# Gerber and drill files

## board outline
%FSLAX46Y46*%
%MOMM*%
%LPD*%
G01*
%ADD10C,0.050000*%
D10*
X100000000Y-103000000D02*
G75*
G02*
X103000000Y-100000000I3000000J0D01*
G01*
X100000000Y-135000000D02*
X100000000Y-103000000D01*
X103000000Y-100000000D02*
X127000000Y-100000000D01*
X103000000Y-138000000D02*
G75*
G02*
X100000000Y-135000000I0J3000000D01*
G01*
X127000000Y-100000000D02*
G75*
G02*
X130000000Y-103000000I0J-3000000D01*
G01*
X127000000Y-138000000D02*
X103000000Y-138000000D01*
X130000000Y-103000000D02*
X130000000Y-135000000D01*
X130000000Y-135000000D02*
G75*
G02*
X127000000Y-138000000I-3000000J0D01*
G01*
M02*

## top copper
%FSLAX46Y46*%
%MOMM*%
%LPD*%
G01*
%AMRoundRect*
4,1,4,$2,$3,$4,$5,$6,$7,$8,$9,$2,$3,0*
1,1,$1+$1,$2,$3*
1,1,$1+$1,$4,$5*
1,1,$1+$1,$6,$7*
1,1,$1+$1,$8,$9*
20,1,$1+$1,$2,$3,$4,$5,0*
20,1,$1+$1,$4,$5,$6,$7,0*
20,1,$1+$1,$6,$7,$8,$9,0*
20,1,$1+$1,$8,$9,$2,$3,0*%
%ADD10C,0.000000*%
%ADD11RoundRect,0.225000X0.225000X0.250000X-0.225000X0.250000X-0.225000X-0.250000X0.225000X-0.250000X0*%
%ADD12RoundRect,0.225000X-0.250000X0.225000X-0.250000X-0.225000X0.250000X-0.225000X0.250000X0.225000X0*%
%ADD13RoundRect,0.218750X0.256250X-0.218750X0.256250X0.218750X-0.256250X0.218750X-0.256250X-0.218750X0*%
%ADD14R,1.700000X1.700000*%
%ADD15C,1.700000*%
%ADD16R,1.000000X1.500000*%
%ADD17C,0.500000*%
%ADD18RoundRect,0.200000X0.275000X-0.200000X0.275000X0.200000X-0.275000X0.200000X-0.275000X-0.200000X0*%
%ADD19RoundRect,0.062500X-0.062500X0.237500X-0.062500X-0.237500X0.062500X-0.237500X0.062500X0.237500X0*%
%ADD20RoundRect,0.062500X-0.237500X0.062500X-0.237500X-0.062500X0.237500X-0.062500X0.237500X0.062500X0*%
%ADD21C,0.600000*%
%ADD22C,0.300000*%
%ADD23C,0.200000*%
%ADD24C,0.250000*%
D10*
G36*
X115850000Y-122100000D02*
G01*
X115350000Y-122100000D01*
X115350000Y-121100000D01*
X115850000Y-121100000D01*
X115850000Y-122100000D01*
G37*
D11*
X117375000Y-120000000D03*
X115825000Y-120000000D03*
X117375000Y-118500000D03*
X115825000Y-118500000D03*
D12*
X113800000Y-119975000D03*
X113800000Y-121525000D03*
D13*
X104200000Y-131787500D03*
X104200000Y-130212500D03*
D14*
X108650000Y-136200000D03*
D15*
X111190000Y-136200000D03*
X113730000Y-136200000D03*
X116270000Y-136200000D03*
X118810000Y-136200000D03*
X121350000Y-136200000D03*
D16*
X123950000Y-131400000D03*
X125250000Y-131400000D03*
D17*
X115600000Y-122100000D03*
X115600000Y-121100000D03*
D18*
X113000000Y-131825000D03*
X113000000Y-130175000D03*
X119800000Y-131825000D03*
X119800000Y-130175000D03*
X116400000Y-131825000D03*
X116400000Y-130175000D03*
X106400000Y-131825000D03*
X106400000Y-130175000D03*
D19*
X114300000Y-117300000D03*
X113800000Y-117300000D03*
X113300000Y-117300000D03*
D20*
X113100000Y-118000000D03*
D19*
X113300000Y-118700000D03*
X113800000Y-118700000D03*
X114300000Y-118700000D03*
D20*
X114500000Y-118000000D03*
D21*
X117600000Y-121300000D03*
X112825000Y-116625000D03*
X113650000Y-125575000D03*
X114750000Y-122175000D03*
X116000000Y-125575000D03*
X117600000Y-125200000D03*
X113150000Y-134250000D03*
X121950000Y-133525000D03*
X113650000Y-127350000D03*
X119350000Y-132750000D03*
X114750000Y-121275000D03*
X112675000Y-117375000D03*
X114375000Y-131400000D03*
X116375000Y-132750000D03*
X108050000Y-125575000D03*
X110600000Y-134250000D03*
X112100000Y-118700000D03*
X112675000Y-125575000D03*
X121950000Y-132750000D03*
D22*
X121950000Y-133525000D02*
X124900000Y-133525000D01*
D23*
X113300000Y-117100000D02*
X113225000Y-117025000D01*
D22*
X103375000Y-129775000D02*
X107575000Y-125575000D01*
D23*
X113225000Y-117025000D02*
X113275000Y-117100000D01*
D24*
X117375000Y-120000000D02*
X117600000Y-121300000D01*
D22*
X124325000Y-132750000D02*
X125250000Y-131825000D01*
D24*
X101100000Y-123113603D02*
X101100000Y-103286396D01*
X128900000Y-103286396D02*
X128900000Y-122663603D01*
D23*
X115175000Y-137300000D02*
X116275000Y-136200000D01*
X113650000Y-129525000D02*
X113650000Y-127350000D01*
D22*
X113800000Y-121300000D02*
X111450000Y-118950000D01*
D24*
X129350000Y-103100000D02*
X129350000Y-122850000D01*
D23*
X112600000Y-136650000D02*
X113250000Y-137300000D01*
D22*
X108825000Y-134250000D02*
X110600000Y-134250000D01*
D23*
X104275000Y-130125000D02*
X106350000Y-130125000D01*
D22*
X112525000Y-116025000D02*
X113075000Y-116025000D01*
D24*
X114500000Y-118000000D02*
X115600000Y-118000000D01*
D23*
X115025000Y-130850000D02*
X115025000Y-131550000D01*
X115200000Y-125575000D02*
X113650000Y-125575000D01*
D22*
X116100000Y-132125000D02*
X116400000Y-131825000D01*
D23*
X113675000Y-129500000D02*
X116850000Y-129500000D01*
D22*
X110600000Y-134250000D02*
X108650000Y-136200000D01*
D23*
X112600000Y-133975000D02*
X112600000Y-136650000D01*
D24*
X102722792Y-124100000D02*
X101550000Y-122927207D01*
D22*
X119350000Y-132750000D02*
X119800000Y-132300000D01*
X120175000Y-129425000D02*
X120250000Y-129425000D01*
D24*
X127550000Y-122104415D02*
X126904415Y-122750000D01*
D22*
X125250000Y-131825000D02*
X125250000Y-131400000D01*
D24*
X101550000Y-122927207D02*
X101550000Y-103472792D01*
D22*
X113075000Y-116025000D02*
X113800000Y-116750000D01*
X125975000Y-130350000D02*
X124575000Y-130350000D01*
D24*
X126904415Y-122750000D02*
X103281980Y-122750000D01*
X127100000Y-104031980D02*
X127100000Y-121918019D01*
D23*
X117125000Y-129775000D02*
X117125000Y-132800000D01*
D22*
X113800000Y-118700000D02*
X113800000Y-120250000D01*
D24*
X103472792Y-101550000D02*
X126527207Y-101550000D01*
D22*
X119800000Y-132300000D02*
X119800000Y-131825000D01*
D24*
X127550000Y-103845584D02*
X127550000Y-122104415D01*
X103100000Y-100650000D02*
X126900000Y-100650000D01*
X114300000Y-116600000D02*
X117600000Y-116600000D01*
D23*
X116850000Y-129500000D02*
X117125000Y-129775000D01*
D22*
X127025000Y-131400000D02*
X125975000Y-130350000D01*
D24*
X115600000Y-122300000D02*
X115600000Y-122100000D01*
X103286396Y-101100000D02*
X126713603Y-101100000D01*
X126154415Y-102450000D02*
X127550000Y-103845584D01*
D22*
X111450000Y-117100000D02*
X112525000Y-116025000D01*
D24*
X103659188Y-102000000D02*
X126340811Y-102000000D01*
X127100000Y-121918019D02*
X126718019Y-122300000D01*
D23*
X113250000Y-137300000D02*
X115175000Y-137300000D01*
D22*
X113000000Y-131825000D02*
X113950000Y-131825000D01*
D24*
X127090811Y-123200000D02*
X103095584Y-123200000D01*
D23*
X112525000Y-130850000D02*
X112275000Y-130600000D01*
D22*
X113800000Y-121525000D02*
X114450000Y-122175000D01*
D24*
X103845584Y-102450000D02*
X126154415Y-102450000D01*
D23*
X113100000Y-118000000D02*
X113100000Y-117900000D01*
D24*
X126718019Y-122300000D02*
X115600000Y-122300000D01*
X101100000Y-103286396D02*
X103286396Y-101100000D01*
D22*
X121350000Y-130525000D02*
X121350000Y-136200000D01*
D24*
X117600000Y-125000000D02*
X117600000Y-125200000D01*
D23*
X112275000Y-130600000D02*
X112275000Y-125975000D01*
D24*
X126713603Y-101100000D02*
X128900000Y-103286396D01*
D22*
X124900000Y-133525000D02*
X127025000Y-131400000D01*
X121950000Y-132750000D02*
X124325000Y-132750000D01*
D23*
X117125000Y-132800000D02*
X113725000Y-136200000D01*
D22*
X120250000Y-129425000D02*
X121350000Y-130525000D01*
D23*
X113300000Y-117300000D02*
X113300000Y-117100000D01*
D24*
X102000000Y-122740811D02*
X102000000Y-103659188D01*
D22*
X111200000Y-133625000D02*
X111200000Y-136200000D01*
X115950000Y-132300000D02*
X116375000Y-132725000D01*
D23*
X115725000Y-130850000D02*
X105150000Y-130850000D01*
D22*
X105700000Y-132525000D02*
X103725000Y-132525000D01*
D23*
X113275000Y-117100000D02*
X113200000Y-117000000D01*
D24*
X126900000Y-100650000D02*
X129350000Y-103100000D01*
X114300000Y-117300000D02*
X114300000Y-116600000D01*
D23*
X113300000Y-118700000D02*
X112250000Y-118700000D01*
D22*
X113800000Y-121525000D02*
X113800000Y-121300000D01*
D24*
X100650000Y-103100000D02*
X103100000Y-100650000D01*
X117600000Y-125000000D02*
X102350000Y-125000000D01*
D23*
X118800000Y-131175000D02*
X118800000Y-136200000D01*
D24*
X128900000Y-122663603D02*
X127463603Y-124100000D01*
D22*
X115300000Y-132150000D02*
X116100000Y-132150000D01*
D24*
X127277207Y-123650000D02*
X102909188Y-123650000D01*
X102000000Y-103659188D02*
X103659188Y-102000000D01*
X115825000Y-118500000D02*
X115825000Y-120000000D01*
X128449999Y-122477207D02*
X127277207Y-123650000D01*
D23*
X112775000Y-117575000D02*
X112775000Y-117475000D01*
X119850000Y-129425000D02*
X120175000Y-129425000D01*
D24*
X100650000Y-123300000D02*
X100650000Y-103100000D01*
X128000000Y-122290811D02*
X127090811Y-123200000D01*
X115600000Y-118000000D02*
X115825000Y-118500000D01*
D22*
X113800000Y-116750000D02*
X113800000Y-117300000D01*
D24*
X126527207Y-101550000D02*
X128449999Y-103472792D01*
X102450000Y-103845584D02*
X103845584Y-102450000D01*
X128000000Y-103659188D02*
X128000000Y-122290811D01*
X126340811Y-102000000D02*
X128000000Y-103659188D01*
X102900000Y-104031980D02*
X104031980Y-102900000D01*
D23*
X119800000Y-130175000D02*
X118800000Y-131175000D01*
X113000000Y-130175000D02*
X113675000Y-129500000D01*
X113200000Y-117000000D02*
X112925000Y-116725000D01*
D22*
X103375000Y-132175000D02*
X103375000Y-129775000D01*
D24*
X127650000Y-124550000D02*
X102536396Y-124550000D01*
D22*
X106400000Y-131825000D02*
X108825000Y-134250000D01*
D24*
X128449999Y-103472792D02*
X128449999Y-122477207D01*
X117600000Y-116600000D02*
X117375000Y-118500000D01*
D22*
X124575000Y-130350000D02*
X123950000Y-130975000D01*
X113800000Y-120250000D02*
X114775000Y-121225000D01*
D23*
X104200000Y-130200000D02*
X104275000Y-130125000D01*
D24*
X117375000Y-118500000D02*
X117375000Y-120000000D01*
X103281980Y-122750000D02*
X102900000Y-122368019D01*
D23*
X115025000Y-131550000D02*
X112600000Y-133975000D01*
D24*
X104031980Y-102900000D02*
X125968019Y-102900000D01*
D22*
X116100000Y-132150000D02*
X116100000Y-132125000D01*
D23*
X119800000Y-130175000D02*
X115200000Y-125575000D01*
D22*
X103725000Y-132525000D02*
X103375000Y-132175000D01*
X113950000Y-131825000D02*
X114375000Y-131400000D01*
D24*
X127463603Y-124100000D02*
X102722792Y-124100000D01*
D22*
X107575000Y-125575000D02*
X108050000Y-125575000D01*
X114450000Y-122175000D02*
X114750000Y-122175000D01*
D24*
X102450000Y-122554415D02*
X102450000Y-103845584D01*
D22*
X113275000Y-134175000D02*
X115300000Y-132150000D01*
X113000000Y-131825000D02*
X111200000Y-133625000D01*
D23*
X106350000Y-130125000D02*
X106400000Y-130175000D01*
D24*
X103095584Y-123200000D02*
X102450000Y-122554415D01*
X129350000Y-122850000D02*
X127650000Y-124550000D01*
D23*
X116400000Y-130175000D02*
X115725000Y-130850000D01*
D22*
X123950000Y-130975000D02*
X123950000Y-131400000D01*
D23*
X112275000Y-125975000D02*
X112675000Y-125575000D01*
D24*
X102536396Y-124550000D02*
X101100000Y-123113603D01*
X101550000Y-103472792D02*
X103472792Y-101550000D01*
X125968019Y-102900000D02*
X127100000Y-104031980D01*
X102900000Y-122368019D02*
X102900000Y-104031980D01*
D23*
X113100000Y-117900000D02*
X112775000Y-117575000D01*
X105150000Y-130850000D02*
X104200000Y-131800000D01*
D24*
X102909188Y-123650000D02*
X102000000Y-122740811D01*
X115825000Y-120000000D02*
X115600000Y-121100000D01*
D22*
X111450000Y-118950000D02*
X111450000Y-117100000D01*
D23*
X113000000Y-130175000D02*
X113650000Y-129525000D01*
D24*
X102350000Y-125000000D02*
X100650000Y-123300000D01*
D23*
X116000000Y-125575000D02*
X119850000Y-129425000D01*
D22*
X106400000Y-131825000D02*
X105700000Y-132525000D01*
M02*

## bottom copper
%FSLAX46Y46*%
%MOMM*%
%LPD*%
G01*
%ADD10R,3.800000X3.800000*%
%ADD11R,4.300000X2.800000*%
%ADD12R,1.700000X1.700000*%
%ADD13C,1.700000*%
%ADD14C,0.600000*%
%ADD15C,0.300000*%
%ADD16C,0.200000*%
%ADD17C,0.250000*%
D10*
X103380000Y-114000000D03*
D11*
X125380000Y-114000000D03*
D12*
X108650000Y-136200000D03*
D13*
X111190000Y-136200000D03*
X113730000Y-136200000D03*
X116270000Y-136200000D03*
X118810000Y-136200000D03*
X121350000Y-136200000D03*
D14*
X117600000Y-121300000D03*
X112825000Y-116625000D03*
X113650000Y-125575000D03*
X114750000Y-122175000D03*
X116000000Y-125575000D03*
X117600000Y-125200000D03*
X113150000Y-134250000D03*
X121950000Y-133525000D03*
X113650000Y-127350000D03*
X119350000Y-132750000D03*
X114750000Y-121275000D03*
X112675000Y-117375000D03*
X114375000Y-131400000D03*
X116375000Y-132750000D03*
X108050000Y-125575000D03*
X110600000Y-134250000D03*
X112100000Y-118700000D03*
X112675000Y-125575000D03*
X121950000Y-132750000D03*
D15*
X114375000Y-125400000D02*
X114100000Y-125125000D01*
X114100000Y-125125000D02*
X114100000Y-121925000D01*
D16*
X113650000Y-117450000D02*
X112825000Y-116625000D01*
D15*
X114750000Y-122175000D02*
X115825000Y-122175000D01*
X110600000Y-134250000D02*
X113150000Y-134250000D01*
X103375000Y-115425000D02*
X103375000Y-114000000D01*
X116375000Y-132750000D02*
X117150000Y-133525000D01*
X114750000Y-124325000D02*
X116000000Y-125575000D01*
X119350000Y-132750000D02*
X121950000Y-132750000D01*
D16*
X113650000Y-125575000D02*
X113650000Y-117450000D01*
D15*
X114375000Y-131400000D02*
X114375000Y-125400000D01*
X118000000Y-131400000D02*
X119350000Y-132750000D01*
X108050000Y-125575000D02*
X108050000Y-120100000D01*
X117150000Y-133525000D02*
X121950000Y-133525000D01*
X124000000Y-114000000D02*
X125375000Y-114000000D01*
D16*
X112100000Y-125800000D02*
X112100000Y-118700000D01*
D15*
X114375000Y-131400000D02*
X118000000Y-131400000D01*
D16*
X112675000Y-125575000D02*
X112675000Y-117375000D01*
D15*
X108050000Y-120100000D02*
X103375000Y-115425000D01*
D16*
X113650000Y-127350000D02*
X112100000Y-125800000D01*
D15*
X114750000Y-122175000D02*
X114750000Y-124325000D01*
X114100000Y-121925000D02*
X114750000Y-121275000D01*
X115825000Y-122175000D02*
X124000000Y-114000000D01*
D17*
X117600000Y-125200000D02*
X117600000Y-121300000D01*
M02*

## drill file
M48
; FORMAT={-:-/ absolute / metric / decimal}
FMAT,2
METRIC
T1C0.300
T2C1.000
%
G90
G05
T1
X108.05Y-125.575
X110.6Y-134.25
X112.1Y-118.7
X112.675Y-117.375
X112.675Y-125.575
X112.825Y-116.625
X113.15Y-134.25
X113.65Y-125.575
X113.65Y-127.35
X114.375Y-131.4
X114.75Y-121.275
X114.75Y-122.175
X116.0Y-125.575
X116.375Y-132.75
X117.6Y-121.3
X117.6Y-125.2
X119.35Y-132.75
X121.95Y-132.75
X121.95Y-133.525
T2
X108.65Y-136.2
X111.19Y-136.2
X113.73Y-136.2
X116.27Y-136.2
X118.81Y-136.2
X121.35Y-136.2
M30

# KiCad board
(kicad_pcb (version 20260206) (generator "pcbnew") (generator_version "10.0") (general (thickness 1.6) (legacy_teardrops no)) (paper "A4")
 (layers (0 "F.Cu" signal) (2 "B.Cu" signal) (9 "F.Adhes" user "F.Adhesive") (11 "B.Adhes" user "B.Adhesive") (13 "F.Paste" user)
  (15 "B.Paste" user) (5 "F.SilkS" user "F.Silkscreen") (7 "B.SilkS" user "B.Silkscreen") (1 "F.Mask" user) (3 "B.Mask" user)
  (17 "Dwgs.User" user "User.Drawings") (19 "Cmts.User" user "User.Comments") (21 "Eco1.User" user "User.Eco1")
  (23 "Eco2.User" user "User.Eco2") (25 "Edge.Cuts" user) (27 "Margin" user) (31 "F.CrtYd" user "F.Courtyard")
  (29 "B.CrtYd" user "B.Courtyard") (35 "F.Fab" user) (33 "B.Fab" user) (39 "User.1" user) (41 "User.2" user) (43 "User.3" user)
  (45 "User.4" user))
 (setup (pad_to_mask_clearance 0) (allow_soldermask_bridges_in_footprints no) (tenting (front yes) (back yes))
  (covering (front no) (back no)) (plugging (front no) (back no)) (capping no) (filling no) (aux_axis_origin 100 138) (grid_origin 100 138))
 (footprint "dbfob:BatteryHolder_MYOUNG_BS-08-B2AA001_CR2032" (layer "B.Cu") (at 114.4 114 180)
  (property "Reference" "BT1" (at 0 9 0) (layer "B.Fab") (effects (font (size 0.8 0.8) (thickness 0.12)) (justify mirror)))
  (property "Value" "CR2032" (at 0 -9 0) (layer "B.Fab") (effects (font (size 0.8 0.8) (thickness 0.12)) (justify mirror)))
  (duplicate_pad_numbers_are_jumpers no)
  (pad "1" smd rect (at 11.02 0 180) (size 3.8 3.8) (layers "B.Cu" "B.Mask" "B.Paste") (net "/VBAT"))
  (pad "2" smd rect (at -10.98 0 180) (size 4.3 2.8) (layers "B.Cu" "B.Mask" "B.Paste") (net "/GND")))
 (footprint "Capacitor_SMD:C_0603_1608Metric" (layer "F.Cu") (at 116.6 120 180)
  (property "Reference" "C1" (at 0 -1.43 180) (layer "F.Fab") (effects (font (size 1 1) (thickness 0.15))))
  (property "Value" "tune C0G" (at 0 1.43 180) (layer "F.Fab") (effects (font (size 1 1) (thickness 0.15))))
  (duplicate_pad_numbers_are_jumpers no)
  (pad "1" smd roundrect (at -0.775 0 180) (size 0.9 0.95) (layers "F.Cu" "F.Mask" "F.Paste") (roundrect_rratio 0.25) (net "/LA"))
  (pad "2" smd roundrect (at 0.775 0 180) (size 0.9 0.95) (layers "F.Cu" "F.Mask" "F.Paste") (roundrect_rratio 0.25) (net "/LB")))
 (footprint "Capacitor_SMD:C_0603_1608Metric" (layer "F.Cu") (at 116.6 118.5 180)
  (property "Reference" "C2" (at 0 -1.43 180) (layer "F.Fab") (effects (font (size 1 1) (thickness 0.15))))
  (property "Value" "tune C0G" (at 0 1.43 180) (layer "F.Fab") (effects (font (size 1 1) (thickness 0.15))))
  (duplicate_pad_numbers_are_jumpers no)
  (pad "1" smd roundrect (at -0.775 0 180) (size 0.9 0.95) (layers "F.Cu" "F.Mask" "F.Paste") (roundrect_rratio 0.25) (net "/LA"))
  (pad "2" smd roundrect (at 0.775 0 180) (size 0.9 0.95) (layers "F.Cu" "F.Mask" "F.Paste") (roundrect_rratio 0.25) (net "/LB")))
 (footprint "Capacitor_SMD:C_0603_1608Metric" (layer "F.Cu") (at 113.8 120.75 -90)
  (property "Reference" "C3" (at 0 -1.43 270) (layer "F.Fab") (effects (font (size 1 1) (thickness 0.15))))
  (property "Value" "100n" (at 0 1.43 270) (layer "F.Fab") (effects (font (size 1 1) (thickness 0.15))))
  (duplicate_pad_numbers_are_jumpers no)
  (pad "1" smd roundrect (at -0.775 0 270) (size 0.9 0.95) (layers "F.Cu" "F.Mask" "F.Paste") (roundrect_rratio 0.25) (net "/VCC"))
  (pad "2" smd roundrect (at 0.775 0 270) (size 0.9 0.95) (layers "F.Cu" "F.Mask" "F.Paste") (roundrect_rratio 0.25) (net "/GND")))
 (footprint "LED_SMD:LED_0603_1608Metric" (layer "F.Cu") (at 104.2 131 90)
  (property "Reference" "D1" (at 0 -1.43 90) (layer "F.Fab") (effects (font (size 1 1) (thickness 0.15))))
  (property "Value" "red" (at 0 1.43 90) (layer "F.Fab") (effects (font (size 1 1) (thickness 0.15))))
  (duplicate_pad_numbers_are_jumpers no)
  (pad "1" smd roundrect (at -0.7875 0 90) (size 0.875 0.95) (layers "F.Cu" "F.Mask" "F.Paste") (roundrect_rratio 0.25) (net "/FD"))
  (pad "2" smd roundrect (at 0.7875 0 90) (size 0.875 0.95) (layers "F.Cu" "F.Mask" "F.Paste") (roundrect_rratio 0.25) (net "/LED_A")))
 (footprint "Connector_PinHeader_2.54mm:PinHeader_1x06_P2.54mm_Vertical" (layer "F.Cu") (at 108.65 136.2 90)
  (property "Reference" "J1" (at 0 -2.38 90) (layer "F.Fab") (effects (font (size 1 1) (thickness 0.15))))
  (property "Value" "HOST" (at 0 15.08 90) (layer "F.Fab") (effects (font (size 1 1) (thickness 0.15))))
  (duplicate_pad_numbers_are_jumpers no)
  (pad "1" thru_hole rect (at 0 0 90) (size 1.7 1.7) (drill 1) (layers "*.Cu" "*.Mask") (remove_unused_layers no) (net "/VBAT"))
  (pad "2" thru_hole circle (at 0 2.54 90) (size 1.7 1.7) (drill 1) (layers "*.Cu" "*.Mask") (remove_unused_layers no) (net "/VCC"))
  (pad "3" thru_hole circle (at 0 5.08 90) (size 1.7 1.7) (drill 1) (layers "*.Cu" "*.Mask") (remove_unused_layers no) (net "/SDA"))
  (pad "4" thru_hole circle (at 0 7.62 90) (size 1.7 1.7) (drill 1) (layers "*.Cu" "*.Mask") (remove_unused_layers no) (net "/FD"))
  (pad "5" thru_hole circle (at 0 10.16 90) (size 1.7 1.7) (drill 1) (layers "*.Cu" "*.Mask") (remove_unused_layers no) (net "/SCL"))
  (pad "6" thru_hole circle (at 0 12.7 90) (size 1.7 1.7) (drill 1) (layers "*.Cu" "*.Mask") (remove_unused_layers no) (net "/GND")))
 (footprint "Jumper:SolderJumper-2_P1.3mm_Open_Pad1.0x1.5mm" (layer "F.Cu") (at 124.6 131.4)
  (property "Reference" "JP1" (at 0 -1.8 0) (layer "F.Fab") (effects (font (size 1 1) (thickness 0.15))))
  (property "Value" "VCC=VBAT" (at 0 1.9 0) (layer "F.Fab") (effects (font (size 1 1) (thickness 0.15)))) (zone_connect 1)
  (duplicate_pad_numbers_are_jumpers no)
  (pad "1" smd rect (at -0.65 0) (size 1 1.5) (layers "F.Cu" "F.Mask") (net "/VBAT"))
  (pad "2" smd rect (at 0.65 0) (size 1 1.5) (layers "F.Cu" "F.Mask") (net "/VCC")))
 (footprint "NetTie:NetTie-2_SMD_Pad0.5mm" (layer "F.Cu") (at 115.6 121.6 90)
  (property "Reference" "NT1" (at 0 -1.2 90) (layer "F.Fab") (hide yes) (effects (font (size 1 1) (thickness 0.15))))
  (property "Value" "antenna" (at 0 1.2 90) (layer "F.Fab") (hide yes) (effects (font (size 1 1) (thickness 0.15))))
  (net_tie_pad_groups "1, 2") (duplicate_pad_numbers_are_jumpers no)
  (fp_poly (pts (xy -0.5 -0.25) (xy 0.5 -0.25) (xy 0.5 0.25) (xy -0.5 0.25)) (stroke (width 0) (type solid)) (fill yes) (layer "F.Cu"))
  (pad "1" smd circle (at -0.5 0 90) (size 0.5 0.5) (layers "F.Cu") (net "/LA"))
  (pad "2" smd circle (at 0.5 0 90) (size 0.5 0.5) (layers "F.Cu") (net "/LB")))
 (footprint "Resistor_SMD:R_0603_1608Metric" (layer "F.Cu") (at 113 131 90)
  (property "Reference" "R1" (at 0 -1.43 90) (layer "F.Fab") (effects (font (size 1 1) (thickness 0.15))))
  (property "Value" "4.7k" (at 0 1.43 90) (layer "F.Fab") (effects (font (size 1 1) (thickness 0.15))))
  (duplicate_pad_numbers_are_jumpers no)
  (pad "1" smd roundrect (at -0.825 0 90) (size 0.8 0.95) (layers "F.Cu" "F.Mask" "F.Paste") (roundrect_rratio 0.25) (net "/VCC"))
  (pad "2" smd roundrect (at 0.825 0 90) (size 0.8 0.95) (layers "F.Cu" "F.Mask" "F.Paste") (roundrect_rratio 0.25) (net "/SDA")))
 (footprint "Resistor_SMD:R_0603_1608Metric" (layer "F.Cu") (at 119.8 131 90)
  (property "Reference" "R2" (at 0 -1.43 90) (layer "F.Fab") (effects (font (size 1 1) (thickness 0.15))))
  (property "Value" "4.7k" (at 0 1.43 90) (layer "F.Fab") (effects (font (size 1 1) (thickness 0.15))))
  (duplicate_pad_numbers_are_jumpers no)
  (pad "1" smd roundrect (at -0.825 0 90) (size 0.8 0.95) (layers "F.Cu" "F.Mask" "F.Paste") (roundrect_rratio 0.25) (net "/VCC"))
  (pad "2" smd roundrect (at 0.825 0 90) (size 0.8 0.95) (layers "F.Cu" "F.Mask" "F.Paste") (roundrect_rratio 0.25) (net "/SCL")))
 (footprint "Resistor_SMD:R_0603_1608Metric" (layer "F.Cu") (at 116.4 131 90)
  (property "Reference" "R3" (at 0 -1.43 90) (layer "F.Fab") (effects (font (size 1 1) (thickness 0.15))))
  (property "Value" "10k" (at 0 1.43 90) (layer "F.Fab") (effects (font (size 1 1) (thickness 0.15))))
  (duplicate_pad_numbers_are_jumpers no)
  (pad "1" smd roundrect (at -0.825 0 90) (size 0.8 0.95) (layers "F.Cu" "F.Mask" "F.Paste") (roundrect_rratio 0.25) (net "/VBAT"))
  (pad "2" smd roundrect (at 0.825 0 90) (size 0.8 0.95) (layers "F.Cu" "F.Mask" "F.Paste") (roundrect_rratio 0.25) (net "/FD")))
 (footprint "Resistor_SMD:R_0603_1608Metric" (layer "F.Cu") (at 106.4 131 90)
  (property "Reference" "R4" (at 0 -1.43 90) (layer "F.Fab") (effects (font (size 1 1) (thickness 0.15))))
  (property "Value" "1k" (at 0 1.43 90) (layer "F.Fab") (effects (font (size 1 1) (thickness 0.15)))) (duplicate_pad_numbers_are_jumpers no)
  (pad "1" smd roundrect (at -0.825 0 90) (size 0.8 0.95) (layers "F.Cu" "F.Mask" "F.Paste") (roundrect_rratio 0.25) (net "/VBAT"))
  (pad "2" smd roundrect (at 0.825 0 90) (size 0.8 0.95) (layers "F.Cu" "F.Mask" "F.Paste") (roundrect_rratio 0.25) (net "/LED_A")))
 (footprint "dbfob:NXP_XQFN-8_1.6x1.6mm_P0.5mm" (layer "F.Cu") (at 113.8 118 -90)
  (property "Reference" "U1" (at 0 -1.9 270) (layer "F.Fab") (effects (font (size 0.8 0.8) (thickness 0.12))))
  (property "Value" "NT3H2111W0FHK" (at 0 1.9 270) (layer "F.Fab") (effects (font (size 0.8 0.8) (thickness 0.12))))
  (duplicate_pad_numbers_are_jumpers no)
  (pad "1" smd roundrect (at -0.7 -0.5 270) (size 0.6 0.25) (layers "F.Cu" "F.Mask" "F.Paste") (roundrect_rratio 0.25) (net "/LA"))
  (pad "2" smd roundrect (at -0.7 0 270) (size 0.6 0.25) (layers "F.Cu" "F.Mask" "F.Paste") (roundrect_rratio 0.25) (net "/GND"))
  (pad "3" smd roundrect (at -0.7 0.5 270) (size 0.6 0.25) (layers "F.Cu" "F.Mask" "F.Paste") (roundrect_rratio 0.25) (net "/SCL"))
  (pad "4" smd roundrect (at 0 0.7 270) (size 0.25 0.6) (layers "F.Cu" "F.Mask" "F.Paste") (roundrect_rratio 0.25) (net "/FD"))
  (pad "5" smd roundrect (at 0.7 0.5 270) (size 0.6 0.25) (layers "F.Cu" "F.Mask" "F.Paste") (roundrect_rratio 0.25) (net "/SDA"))
  (pad "6" smd roundrect (at 0.7 0 270) (size 0.6 0.25) (layers "F.Cu" "F.Mask" "F.Paste") (roundrect_rratio 0.25) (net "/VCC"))
  (pad "7" smd roundrect (at 0.7 -0.5 270) (size 0.6 0.25) (layers "F.Cu" "F.Mask" "F.Paste") (roundrect_rratio 0.25)
   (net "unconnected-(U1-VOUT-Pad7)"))
  (pad "8" smd roundrect (at 0 -0.7 270) (size 0.25 0.6) (layers "F.Cu" "F.Mask" "F.Paste") (roundrect_rratio 0.25) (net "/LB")))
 (gr_arc (start 100 103) (mid 100.878679 100.878679) (end 103 100) (stroke (width 0.05) (type default)) (layer "Edge.Cuts"))
 (gr_line (start 100 135) (end 100 103) (stroke (width 0.05) (type default)) (layer "Edge.Cuts"))
 (gr_line (start 103 100) (end 127 100) (stroke (width 0.05) (type default)) (layer "Edge.Cuts"))
 (gr_arc (start 103 138) (mid 100.878679 137.12132) (end 100 135) (stroke (width 0.05) (type default)) (layer "Edge.Cuts"))
 (gr_arc (start 127 100) (mid 129.12132 100.878679) (end 130 103) (stroke (width 0.05) (type default)) (layer "Edge.Cuts"))
 (gr_line (start 127 138) (end 103 138) (stroke (width 0.05) (type default)) (layer "Edge.Cuts"))
 (gr_line (start 130 103) (end 130 135) (stroke (width 0.05) (type default)) (layer "Edge.Cuts"))
 (gr_arc (start 130 135) (mid 129.12132 137.12132) (end 127 138) (stroke (width 0.05) (type default)) (layer "Edge.Cuts"))
 (segment (start 121.950000 133.525000) (end 124.900000 133.525000) (width 0.3) (layer "F.Cu") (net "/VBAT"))
 (segment (start 113.300000 117.100000) (end 113.225000 117.025000) (width 0.2) (layer "F.Cu") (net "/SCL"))
 (segment (start 103.375000 129.775000) (end 107.575000 125.575000) (width 0.3) (layer "F.Cu") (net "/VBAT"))
 (segment (start 113.225000 117.025000) (end 113.275000 117.100000) (width 0.2) (layer "F.Cu") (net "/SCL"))
 (segment (start 114.375000 125.400000) (end 114.100000 125.125000) (width 0.3) (layer "B.Cu") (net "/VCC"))
 (segment (start 117.375 120) (end 117.6 121.3) (width 0.25) (layer "F.Cu") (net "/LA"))
 (segment (start 124.325000 132.750000) (end 125.250000 131.825000) (width 0.3) (layer "F.Cu") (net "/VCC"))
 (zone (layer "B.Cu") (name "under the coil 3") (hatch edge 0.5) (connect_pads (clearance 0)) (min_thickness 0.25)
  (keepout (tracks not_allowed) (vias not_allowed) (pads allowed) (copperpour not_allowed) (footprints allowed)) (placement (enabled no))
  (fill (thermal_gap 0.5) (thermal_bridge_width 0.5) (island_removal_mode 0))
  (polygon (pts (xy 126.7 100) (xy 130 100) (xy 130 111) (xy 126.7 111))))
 (via (at 117.6 121.3) (size 0.6) (drill 0.3) (layers "F.Cu" "B.Cu") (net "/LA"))
 (segment (start 101.1 123.113603) (end 101.1 103.286396) (width 0.25) (layer "F.Cu") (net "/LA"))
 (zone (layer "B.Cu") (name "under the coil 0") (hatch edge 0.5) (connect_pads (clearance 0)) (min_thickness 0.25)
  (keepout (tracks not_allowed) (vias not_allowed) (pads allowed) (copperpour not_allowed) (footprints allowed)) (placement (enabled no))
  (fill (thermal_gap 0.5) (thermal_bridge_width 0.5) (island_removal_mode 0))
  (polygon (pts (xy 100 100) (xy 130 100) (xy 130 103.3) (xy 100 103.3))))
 (segment (start 128.9 103.286396) (end 128.9 122.663603) (width 0.25) (layer "F.Cu") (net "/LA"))
 (segment (start 115.175000 137.300000) (end 116.275000 136.200000) (width 0.2) (layer "F.Cu") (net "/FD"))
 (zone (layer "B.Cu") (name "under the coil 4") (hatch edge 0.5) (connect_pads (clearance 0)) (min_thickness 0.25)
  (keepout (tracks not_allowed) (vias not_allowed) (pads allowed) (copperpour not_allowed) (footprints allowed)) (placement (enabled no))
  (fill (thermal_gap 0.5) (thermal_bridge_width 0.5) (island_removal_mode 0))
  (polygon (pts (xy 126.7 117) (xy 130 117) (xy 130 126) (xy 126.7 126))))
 (segment (start 113.650000 129.525000) (end 113.650000 127.350000) (width 0.2) (layer "F.Cu") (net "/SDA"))
 (segment (start 114.100000 125.125000) (end 114.100000 121.925000) (width 0.3) (layer "B.Cu") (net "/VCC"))
 (segment (start 113.800000 121.300000) (end 111.450000 118.950000) (width 0.3) (layer "F.Cu") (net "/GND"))
 (segment (start 129.35 103.1) (end 129.35 122.85) (width 0.25) (layer "F.Cu") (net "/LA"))
 (segment (start 112.600000 136.650000) (end 113.250000 137.300000) (width 0.2) (layer "F.Cu") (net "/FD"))
 (segment (start 108.825000 134.250000) (end 110.600000 134.250000) (width 0.3) (layer "F.Cu") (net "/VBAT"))
 (segment (start 104.275000 130.125000) (end 106.350000 130.125000) (width 0.2) (layer "F.Cu") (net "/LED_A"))
 (segment (start 112.525000 116.025000) (end 113.075000 116.025000) (width 0.3) (layer "F.Cu") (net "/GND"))
 (segment (start 114.5 118) (end 115.6 118) (width 0.25) (layer "F.Cu") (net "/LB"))
 (segment (start 115.025000 130.850000) (end 115.025000 131.550000) (width 0.2) (layer "F.Cu") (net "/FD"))
 (via (at 112.825000 116.625000) (size 0.6) (drill 0.3) (layers "F.Cu" "B.Cu") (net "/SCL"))
 (segment (start 115.200000 125.575000) (end 113.650000 125.575000) (width 0.2) (layer "F.Cu") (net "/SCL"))
 (segment (start 116.100000 132.125000) (end 116.400000 131.825000) (width 0.3) (layer "F.Cu") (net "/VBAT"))
 (segment (start 113.675000 129.500000) (end 116.850000 129.500000) (width 0.2) (layer "F.Cu") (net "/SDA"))
 (segment (start 110.600000 134.250000) (end 108.650000 136.200000) (width 0.3) (layer "F.Cu") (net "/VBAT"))
 (segment (start 112.600000 133.975000) (end 112.600000 136.650000) (width 0.2) (layer "F.Cu") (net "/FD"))
 (via (at 113.650000 125.575000) (size 0.6) (drill 0.3) (layers "F.Cu" "B.Cu") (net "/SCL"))
 (segment (start 102.722792 124.1) (end 101.55 122.927207) (width 0.25) (layer "F.Cu") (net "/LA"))
 (segment (start 113.650000 117.450000) (end 112.825000 116.625000) (width 0.2) (layer "B.Cu") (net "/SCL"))
 (segment (start 119.350000 132.750000) (end 119.800000 132.300000) (width 0.3) (layer "F.Cu") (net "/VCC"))
 (segment (start 120.175000 129.425000) (end 120.250000 129.425000) (width 0.3) (layer "F.Cu") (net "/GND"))
 (segment (start 127.55 122.104415) (end 126.904415 122.75) (width 0.25) (layer "F.Cu") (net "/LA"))
 (via (at 114.750000 122.175000) (size 0.6) (drill 0.3) (layers "F.Cu" "B.Cu") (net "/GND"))
 (segment (start 125.250000 131.825000) (end 125.250000 131.400000) (width 0.3) (layer "F.Cu") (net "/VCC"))
 (segment (start 101.55 122.927207) (end 101.55 103.472792) (width 0.25) (layer "F.Cu") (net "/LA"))
 (segment (start 113.075000 116.025000) (end 113.800000 116.750000) (width 0.3) (layer "F.Cu") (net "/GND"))
 (segment (start 125.975000 130.350000) (end 124.575000 130.350000) (width 0.3) (layer "F.Cu") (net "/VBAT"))
 (segment (start 114.750000 122.175000) (end 115.825000 122.175000) (width 0.3) (layer "B.Cu") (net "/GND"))
 (segment (start 126.904415 122.75) (end 103.28198 122.75) (width 0.25) (layer "F.Cu") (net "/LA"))
 (segment (start 127.1 104.03198) (end 127.1 121.918019) (width 0.25) (layer "F.Cu") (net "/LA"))
 (segment (start 117.125000 129.775000) (end 117.125000 132.800000) (width 0.2) (layer "F.Cu") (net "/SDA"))
 (segment (start 113.800000 118.700000) (end 113.800000 120.250000) (width 0.3) (layer "F.Cu") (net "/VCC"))
 (segment (start 103.472792 101.55) (end 126.527207 101.55) (width 0.25) (layer "F.Cu") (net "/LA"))
 (segment (start 119.800000 132.300000) (end 119.800000 131.825000) (width 0.3) (layer "F.Cu") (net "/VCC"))
 (segment (start 127.55 103.845584) (end 127.55 122.104415) (width 0.25) (layer "F.Cu") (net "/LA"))
 (via (at 116.000000 125.575000) (size 0.6) (drill 0.3) (layers "F.Cu" "B.Cu") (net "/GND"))
 (segment (start 110.600000 134.250000) (end 113.150000 134.250000) (width 0.3) (layer "B.Cu") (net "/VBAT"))
 (segment (start 103.1 100.65) (end 126.9 100.65) (width 0.25) (layer "F.Cu") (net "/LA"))
 (via (at 117.6 125.2) (size 0.6) (drill 0.3) (layers "F.Cu" "B.Cu") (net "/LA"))
 (segment (start 114.3 116.6) (end 117.6 116.6) (width 0.25) (layer "F.Cu") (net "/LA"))
 (segment (start 116.850000 129.500000) (end 117.125000 129.775000) (width 0.2) (layer "F.Cu") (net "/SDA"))
 (segment (start 127.025000 131.400000) (end 125.975000 130.350000) (width 0.3) (layer "F.Cu") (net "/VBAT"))
 (segment (start 115.6 122.3) (end 115.6 122.1) (width 0.25) (layer "F.Cu") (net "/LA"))
 (segment (start 103.375000 115.425000) (end 103.375000 114.000000) (width 0.3) (layer "B.Cu") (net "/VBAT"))
 (segment (start 103.286396 101.1) (end 126.713603 101.1) (width 0.25) (layer "F.Cu") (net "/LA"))
 (segment (start 126.154415 102.45) (end 127.55 103.845584) (width 0.25) (layer "F.Cu") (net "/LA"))
 (segment (start 111.450000 117.100000) (end 112.525000 116.025000) (width 0.3) (layer "F.Cu") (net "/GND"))
 (segment (start 103.659188 102) (end 126.340811 102) (width 0.25) (layer "F.Cu") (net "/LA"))
 (via (at 113.150000 134.250000) (size 0.6) (drill 0.3) (layers "F.Cu" "B.Cu") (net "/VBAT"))
 (segment (start 127.1 121.918019) (end 126.718019 122.3) (width 0.25) (layer "F.Cu") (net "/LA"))
 (segment (start 113.250000 137.300000) (end 115.175000 137.300000) (width 0.2) (layer "F.Cu") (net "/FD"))
 (via (at 121.950000 133.525000) (size 0.6) (drill 0.3) (layers "F.Cu" "B.Cu") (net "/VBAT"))
 (segment (start 113.000000 131.825000) (end 113.950000 131.825000) (width 0.3) (layer "F.Cu") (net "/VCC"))
 (segment (start 116.375000 132.750000) (end 117.150000 133.525000) (width 0.3) (layer "B.Cu") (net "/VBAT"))
 (segment (start 127.090811 123.2) (end 103.095584 123.2) (width 0.25) (layer "F.Cu") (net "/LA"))
 (segment (start 112.525000 130.850000) (end 112.275000 130.600000) (width 0.2) (layer "F.Cu") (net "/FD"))
 (via (at 113.650000 127.350000) (size 0.6) (drill 0.3) (layers "F.Cu" "B.Cu") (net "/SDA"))
 (segment (start 114.750000 124.325000) (end 116.000000 125.575000) (width 0.3) (layer "B.Cu") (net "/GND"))
 (segment (start 113.800000 121.525000) (end 114.450000 122.175000) (width 0.3) (layer "F.Cu") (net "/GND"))
 (via (at 119.350000 132.750000) (size 0.6) (drill 0.3) (layers "F.Cu" "B.Cu") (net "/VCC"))
 (segment (start 103.845584 102.45) (end 126.154415 102.45) (width 0.25) (layer "F.Cu") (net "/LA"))
 (segment (start 113.100000 118.000000) (end 113.100000 117.900000) (width 0.2) (layer "F.Cu") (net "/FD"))
 (segment (start 126.718019 122.3) (end 115.6 122.3) (width 0.25) (layer "F.Cu") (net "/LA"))
 (segment (start 101.1 103.286396) (end 103.286396 101.1) (width 0.25) (layer "F.Cu") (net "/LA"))
 (segment (start 121.350000 130.525000) (end 121.350000 136.200000) (width 0.3) (layer "F.Cu") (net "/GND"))
 (segment (start 119.350000 132.750000) (end 121.950000 132.750000) (width 0.3) (layer "B.Cu") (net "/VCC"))
 (segment (start 117.6 125) (end 117.6 125.2) (width 0.25) (layer "F.Cu") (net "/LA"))
 (segment (start 112.275000 130.600000) (end 112.275000 125.975000) (width 0.2) (layer "F.Cu") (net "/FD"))
 (segment (start 113.650000 125.575000) (end 113.650000 117.450000) (width 0.2) (layer "B.Cu") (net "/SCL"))
 (segment (start 126.713603 101.1) (end 128.9 103.286396) (width 0.25) (layer "F.Cu") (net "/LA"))
 (segment (start 124.900000 133.525000) (end 127.025000 131.400000) (width 0.3) (layer "F.Cu") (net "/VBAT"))
 (segment (start 121.950000 132.750000) (end 124.325000 132.750000) (width 0.3) (layer "F.Cu") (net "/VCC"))
 (segment (start 117.125000 132.800000) (end 113.725000 136.200000) (width 0.2) (layer "F.Cu") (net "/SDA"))
 (segment (start 120.250000 129.425000) (end 121.350000 130.525000) (width 0.3) (layer "F.Cu") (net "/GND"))
 (segment (start 113.300000 117.300000) (end 113.300000 117.100000) (width 0.2) (layer "F.Cu") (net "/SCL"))
 (segment (start 102 122.740811) (end 102 103.659188) (width 0.25) (layer "F.Cu") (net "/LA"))
 (segment (start 114.375000 131.400000) (end 114.375000 125.400000) (width 0.3) (layer "B.Cu") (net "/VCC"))
 (segment (start 111.200000 133.625000) (end 111.200000 136.200000) (width 0.3) (layer "F.Cu") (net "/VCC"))
 (segment (start 118.000000 131.400000) (end 119.350000 132.750000) (width 0.3) (layer "B.Cu") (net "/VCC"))
 (segment (start 115.950000 132.300000) (end 116.375000 132.725000) (width 0.3) (layer "F.Cu") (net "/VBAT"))
 (segment (start 115.725000 130.850000) (end 105.150000 130.850000) (width 0.2) (layer "F.Cu") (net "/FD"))
 (segment (start 105.700000 132.525000) (end 103.725000 132.525000) (width 0.3) (layer "F.Cu") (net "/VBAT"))
 (segment (start 113.275000 117.100000) (end 113.200000 117.000000) (width 0.2) (layer "F.Cu") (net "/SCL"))
 (segment (start 126.9 100.65) (end 129.35 103.1) (width 0.25) (layer "F.Cu") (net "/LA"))
 (segment (start 114.3 117.3) (end 114.3 116.6) (width 0.25) (layer "F.Cu") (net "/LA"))
 (segment (start 113.300000 118.700000) (end 112.250000 118.700000) (width 0.2) (layer "F.Cu") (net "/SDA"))
 (segment (start 113.800000 121.525000) (end 113.800000 121.300000) (width 0.3) (layer "F.Cu") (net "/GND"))
 (via (at 114.750000 121.275000) (size 0.6) (drill 0.3) (layers "F.Cu" "B.Cu") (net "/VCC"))
 (segment (start 100.65 103.1) (end 103.1 100.65) (width 0.25) (layer "F.Cu") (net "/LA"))
 (via (at 112.675000 117.375000) (size 0.6) (drill 0.3) (layers "F.Cu" "B.Cu") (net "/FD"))
 (via (at 114.375000 131.400000) (size 0.6) (drill 0.3) (layers "F.Cu" "B.Cu") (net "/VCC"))
 (segment (start 117.6 125) (end 102.35 125) (width 0.25) (layer "F.Cu") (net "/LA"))
 (segment (start 118.800000 131.175000) (end 118.800000 136.200000) (width 0.2) (layer "F.Cu") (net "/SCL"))
 (via (at 116.375000 132.750000) (size 0.6) (drill 0.3) (layers "F.Cu" "B.Cu") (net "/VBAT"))
 (segment (start 108.050000 125.575000) (end 108.050000 120.100000) (width 0.3) (layer "B.Cu") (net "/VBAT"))
 (segment (start 128.9 122.663603) (end 127.463603 124.1) (width 0.25) (layer "F.Cu") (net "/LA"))
 (segment (start 117.150000 133.525000) (end 121.950000 133.525000) (width 0.3) (layer "B.Cu") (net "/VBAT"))
 (segment (start 115.300000 132.150000) (end 116.100000 132.150000) (width 0.3) (layer "F.Cu") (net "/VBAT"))
 (segment (start 124.000000 114.000000) (end 125.375000 114.000000) (width 0.3) (layer "B.Cu") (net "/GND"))
 (via (at 108.050000 125.575000) (size 0.6) (drill 0.3) (layers "F.Cu" "B.Cu") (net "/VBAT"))
 (segment (start 127.277207 123.65) (end 102.909188 123.65) (width 0.25) (layer "F.Cu") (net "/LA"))
 (segment (start 112.100000 125.800000) (end 112.100000 118.700000) (width 0.2) (layer "B.Cu") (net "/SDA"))
 (segment (start 102 103.659188) (end 103.659188 102) (width 0.25) (layer "F.Cu") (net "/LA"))
 (segment (start 115.825 118.5) (end 115.825 120) (width 0.25) (layer "F.Cu") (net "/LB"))
 (segment (start 128.449999 122.477207) (end 127.277207 123.65) (width 0.25) (layer "F.Cu") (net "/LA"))
 (segment (start 112.775000 117.575000) (end 112.775000 117.475000) (width 0.2) (layer "F.Cu") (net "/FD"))
 (segment (start 119.850000 129.425000) (end 120.175000 129.425000) (width 0.2) (layer "F.Cu") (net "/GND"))
 (segment (start 100.65 123.3) (end 100.65 103.1) (width 0.25) (layer "F.Cu") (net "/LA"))
 (segment (start 128 122.290811) (end 127.090811 123.2) (width 0.25) (layer "F.Cu") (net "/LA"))
 (segment (start 115.6 118) (end 115.825 118.5) (width 0.25) (layer "F.Cu") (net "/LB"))
 (via (at 110.600000 134.250000) (size 0.6) (drill 0.3) (layers "F.Cu" "B.Cu") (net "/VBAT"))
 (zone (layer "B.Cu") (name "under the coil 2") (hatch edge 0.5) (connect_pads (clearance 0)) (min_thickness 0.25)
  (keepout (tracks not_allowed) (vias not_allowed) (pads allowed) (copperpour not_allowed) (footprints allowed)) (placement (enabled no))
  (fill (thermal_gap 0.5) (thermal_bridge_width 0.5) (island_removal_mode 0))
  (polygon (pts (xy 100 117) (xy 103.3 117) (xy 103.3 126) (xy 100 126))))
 (segment (start 113.800000 116.750000) (end 113.800000 117.300000) (width 0.3) (layer "F.Cu") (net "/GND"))
 (segment (start 114.375000 131.400000) (end 118.000000 131.400000) (width 0.3) (layer "B.Cu") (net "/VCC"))
 (segment (start 126.527207 101.55) (end 128.449999 103.472792) (width 0.25) (layer "F.Cu") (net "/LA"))
 (segment (start 102.45 103.845584) (end 103.845584 102.45) (width 0.25) (layer "F.Cu") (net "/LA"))
 (segment (start 112.675000 125.575000) (end 112.675000 117.375000) (width 0.2) (layer "B.Cu") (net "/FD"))
 (segment (start 128 103.659188) (end 128 122.290811) (width 0.25) (layer "F.Cu") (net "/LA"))
 (segment (start 126.340811 102) (end 128 103.659188) (width 0.25) (layer "F.Cu") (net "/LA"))
 (segment (start 102.9 104.03198) (end 104.03198 102.9) (width 0.25) (layer "F.Cu") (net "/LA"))
 (segment (start 119.800000 130.175000) (end 118.800000 131.175000) (width 0.2) (layer "F.Cu") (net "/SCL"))
 (segment (start 113.000000 130.175000) (end 113.675000 129.500000) (width 0.2) (layer "F.Cu") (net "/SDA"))
 (segment (start 113.200000 117.000000) (end 112.925000 116.725000) (width 0.2) (layer "F.Cu") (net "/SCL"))
 (segment (start 103.375000 132.175000) (end 103.375000 129.775000) (width 0.3) (layer "F.Cu") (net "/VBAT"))
 (segment (start 127.65 124.55) (end 102.536396 124.55) (width 0.25) (layer "F.Cu") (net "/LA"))
 (segment (start 106.400000 131.825000) (end 108.825000 134.250000) (width 0.3) (layer "F.Cu") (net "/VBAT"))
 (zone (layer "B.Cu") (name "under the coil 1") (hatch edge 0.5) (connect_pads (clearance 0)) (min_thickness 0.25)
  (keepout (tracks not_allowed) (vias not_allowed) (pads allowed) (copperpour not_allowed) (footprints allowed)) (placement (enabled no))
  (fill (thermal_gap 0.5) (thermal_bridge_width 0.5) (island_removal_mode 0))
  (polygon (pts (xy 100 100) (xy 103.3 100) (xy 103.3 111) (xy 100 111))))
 (segment (start 128.449999 103.472792) (end 128.449999 122.477207) (width 0.25) (layer "F.Cu") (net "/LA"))
 (segment (start 117.6 116.6) (end 117.375 118.5) (width 0.25) (layer "F.Cu") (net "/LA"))
 (segment (start 124.575000 130.350000) (end 123.950000 130.975000) (width 0.3) (layer "F.Cu") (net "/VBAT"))
 (segment (start 113.800000 120.250000) (end 114.775000 121.225000) (width 0.3) (layer "F.Cu") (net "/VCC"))
 (segment (start 104.200000 130.200000) (end 104.275000 130.125000) (width 0.2) (layer "F.Cu") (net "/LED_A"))
 (via (at 112.100000 118.700000) (size 0.6) (drill 0.3) (layers "F.Cu" "B.Cu") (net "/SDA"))
 (segment (start 117.375 118.5) (end 117.375 120) (width 0.25) (layer "F.Cu") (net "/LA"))
 (segment (start 103.28198 122.75) (end 102.9 122.368019) (width 0.25) (layer "F.Cu") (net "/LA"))
 (segment (start 115.025000 131.550000) (end 112.600000 133.975000) (width 0.2) (layer "F.Cu") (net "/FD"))
 (segment (start 108.050000 120.100000) (end 103.375000 115.425000) (width 0.3) (layer "B.Cu") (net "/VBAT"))
 (segment (start 113.650000 127.350000) (end 112.100000 125.800000) (width 0.2) (layer "B.Cu") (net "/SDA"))
 (segment (start 104.03198 102.9) (end 125.968019 102.9) (width 0.25) (layer "F.Cu") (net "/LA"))
 (via (at 112.675000 125.575000) (size 0.6) (drill 0.3) (layers "F.Cu" "B.Cu") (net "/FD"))
 (segment (start 116.100000 132.150000) (end 116.100000 132.125000) (width 0.3) (layer "F.Cu") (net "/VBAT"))
 (segment (start 119.800000 130.175000) (end 115.200000 125.575000) (width 0.2) (layer "F.Cu") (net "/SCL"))
 (via (at 121.950000 132.750000) (size 0.6) (drill 0.3) (layers "F.Cu" "B.Cu") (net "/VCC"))
 (segment (start 103.725000 132.525000) (end 103.375000 132.175000) (width 0.3) (layer "F.Cu") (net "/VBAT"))
 (segment (start 114.750000 122.175000) (end 114.750000 124.325000) (width 0.3) (layer "B.Cu") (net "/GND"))
 (segment (start 114.100000 121.925000) (end 114.750000 121.275000) (width 0.3) (layer "B.Cu") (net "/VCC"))
 (segment (start 113.950000 131.825000) (end 114.375000 131.400000) (width 0.3) (layer "F.Cu") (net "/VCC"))
 (segment (start 127.463603 124.1) (end 102.722792 124.1) (width 0.25) (layer "F.Cu") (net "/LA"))
 (segment (start 107.575000 125.575000) (end 108.050000 125.575000) (width 0.3) (layer "F.Cu") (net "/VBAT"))
 (segment (start 114.450000 122.175000) (end 114.750000 122.175000) (width 0.3) (layer "F.Cu") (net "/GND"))
 (segment (start 102.45 122.554415) (end 102.45 103.845584) (width 0.25) (layer "F.Cu") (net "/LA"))
 (segment (start 113.275000 134.175000) (end 115.300000 132.150000) (width 0.3) (layer "F.Cu") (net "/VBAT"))
 (segment (start 113.000000 131.825000) (end 111.200000 133.625000) (width 0.3) (layer "F.Cu") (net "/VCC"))
 (segment (start 106.350000 130.125000) (end 106.400000 130.175000) (width 0.2) (layer "F.Cu") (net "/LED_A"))
 (segment (start 103.095584 123.2) (end 102.45 122.554415) (width 0.25) (layer "F.Cu") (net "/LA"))
 (segment (start 129.35 122.85) (end 127.65 124.55) (width 0.25) (layer "F.Cu") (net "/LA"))
 (segment (start 116.400000 130.175000) (end 115.725000 130.850000) (width 0.2) (layer "F.Cu") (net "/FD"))
 (segment (start 123.950000 130.975000) (end 123.950000 131.400000) (width 0.3) (layer "F.Cu") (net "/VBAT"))
 (segment (start 112.275000 125.975000) (end 112.675000 125.575000) (width 0.2) (layer "F.Cu") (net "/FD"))
 (segment (start 102.536396 124.55) (end 101.1 123.113603) (width 0.25) (layer "F.Cu") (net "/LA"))
 (segment (start 101.55 103.472792) (end 103.472792 101.55) (width 0.25) (layer "F.Cu") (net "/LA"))
 (segment (start 125.968019 102.9) (end 127.1 104.03198) (width 0.25) (layer "F.Cu") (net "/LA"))
 (segment (start 102.9 122.368019) (end 102.9 104.03198) (width 0.25) (layer "F.Cu") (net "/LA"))
 (segment (start 113.100000 117.900000) (end 112.775000 117.575000) (width 0.2) (layer "F.Cu") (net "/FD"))
 (segment (start 105.150000 130.850000) (end 104.200000 131.800000) (width 0.2) (layer "F.Cu") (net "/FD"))
 (segment (start 102.909188 123.65) (end 102 122.740811) (width 0.25) (layer "F.Cu") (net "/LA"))
 (segment (start 115.825 120) (end 115.6 121.1) (width 0.25) (layer "F.Cu") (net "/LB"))
 (segment (start 111.450000 118.950000) (end 111.450000 117.100000) (width 0.3) (layer "F.Cu") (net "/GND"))
 (segment (start 113.000000 130.175000) (end 113.650000 129.525000) (width 0.2) (layer "F.Cu") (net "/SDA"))
 (segment (start 102.35 125) (end 100.65 123.3) (width 0.25) (layer "F.Cu") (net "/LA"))
 (segment (start 116.000000 125.575000) (end 119.850000 129.425000) (width 0.2) (layer "F.Cu") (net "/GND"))
 (segment (start 115.825000 122.175000) (end 124.000000 114.000000) (width 0.3) (layer "B.Cu") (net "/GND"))
 (segment (start 117.6 125.2) (end 117.6 121.3) (width 0.25) (layer "B.Cu") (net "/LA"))
 (segment (start 106.400000 131.825000) (end 105.700000 132.525000) (width 0.3) (layer "F.Cu") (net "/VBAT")))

